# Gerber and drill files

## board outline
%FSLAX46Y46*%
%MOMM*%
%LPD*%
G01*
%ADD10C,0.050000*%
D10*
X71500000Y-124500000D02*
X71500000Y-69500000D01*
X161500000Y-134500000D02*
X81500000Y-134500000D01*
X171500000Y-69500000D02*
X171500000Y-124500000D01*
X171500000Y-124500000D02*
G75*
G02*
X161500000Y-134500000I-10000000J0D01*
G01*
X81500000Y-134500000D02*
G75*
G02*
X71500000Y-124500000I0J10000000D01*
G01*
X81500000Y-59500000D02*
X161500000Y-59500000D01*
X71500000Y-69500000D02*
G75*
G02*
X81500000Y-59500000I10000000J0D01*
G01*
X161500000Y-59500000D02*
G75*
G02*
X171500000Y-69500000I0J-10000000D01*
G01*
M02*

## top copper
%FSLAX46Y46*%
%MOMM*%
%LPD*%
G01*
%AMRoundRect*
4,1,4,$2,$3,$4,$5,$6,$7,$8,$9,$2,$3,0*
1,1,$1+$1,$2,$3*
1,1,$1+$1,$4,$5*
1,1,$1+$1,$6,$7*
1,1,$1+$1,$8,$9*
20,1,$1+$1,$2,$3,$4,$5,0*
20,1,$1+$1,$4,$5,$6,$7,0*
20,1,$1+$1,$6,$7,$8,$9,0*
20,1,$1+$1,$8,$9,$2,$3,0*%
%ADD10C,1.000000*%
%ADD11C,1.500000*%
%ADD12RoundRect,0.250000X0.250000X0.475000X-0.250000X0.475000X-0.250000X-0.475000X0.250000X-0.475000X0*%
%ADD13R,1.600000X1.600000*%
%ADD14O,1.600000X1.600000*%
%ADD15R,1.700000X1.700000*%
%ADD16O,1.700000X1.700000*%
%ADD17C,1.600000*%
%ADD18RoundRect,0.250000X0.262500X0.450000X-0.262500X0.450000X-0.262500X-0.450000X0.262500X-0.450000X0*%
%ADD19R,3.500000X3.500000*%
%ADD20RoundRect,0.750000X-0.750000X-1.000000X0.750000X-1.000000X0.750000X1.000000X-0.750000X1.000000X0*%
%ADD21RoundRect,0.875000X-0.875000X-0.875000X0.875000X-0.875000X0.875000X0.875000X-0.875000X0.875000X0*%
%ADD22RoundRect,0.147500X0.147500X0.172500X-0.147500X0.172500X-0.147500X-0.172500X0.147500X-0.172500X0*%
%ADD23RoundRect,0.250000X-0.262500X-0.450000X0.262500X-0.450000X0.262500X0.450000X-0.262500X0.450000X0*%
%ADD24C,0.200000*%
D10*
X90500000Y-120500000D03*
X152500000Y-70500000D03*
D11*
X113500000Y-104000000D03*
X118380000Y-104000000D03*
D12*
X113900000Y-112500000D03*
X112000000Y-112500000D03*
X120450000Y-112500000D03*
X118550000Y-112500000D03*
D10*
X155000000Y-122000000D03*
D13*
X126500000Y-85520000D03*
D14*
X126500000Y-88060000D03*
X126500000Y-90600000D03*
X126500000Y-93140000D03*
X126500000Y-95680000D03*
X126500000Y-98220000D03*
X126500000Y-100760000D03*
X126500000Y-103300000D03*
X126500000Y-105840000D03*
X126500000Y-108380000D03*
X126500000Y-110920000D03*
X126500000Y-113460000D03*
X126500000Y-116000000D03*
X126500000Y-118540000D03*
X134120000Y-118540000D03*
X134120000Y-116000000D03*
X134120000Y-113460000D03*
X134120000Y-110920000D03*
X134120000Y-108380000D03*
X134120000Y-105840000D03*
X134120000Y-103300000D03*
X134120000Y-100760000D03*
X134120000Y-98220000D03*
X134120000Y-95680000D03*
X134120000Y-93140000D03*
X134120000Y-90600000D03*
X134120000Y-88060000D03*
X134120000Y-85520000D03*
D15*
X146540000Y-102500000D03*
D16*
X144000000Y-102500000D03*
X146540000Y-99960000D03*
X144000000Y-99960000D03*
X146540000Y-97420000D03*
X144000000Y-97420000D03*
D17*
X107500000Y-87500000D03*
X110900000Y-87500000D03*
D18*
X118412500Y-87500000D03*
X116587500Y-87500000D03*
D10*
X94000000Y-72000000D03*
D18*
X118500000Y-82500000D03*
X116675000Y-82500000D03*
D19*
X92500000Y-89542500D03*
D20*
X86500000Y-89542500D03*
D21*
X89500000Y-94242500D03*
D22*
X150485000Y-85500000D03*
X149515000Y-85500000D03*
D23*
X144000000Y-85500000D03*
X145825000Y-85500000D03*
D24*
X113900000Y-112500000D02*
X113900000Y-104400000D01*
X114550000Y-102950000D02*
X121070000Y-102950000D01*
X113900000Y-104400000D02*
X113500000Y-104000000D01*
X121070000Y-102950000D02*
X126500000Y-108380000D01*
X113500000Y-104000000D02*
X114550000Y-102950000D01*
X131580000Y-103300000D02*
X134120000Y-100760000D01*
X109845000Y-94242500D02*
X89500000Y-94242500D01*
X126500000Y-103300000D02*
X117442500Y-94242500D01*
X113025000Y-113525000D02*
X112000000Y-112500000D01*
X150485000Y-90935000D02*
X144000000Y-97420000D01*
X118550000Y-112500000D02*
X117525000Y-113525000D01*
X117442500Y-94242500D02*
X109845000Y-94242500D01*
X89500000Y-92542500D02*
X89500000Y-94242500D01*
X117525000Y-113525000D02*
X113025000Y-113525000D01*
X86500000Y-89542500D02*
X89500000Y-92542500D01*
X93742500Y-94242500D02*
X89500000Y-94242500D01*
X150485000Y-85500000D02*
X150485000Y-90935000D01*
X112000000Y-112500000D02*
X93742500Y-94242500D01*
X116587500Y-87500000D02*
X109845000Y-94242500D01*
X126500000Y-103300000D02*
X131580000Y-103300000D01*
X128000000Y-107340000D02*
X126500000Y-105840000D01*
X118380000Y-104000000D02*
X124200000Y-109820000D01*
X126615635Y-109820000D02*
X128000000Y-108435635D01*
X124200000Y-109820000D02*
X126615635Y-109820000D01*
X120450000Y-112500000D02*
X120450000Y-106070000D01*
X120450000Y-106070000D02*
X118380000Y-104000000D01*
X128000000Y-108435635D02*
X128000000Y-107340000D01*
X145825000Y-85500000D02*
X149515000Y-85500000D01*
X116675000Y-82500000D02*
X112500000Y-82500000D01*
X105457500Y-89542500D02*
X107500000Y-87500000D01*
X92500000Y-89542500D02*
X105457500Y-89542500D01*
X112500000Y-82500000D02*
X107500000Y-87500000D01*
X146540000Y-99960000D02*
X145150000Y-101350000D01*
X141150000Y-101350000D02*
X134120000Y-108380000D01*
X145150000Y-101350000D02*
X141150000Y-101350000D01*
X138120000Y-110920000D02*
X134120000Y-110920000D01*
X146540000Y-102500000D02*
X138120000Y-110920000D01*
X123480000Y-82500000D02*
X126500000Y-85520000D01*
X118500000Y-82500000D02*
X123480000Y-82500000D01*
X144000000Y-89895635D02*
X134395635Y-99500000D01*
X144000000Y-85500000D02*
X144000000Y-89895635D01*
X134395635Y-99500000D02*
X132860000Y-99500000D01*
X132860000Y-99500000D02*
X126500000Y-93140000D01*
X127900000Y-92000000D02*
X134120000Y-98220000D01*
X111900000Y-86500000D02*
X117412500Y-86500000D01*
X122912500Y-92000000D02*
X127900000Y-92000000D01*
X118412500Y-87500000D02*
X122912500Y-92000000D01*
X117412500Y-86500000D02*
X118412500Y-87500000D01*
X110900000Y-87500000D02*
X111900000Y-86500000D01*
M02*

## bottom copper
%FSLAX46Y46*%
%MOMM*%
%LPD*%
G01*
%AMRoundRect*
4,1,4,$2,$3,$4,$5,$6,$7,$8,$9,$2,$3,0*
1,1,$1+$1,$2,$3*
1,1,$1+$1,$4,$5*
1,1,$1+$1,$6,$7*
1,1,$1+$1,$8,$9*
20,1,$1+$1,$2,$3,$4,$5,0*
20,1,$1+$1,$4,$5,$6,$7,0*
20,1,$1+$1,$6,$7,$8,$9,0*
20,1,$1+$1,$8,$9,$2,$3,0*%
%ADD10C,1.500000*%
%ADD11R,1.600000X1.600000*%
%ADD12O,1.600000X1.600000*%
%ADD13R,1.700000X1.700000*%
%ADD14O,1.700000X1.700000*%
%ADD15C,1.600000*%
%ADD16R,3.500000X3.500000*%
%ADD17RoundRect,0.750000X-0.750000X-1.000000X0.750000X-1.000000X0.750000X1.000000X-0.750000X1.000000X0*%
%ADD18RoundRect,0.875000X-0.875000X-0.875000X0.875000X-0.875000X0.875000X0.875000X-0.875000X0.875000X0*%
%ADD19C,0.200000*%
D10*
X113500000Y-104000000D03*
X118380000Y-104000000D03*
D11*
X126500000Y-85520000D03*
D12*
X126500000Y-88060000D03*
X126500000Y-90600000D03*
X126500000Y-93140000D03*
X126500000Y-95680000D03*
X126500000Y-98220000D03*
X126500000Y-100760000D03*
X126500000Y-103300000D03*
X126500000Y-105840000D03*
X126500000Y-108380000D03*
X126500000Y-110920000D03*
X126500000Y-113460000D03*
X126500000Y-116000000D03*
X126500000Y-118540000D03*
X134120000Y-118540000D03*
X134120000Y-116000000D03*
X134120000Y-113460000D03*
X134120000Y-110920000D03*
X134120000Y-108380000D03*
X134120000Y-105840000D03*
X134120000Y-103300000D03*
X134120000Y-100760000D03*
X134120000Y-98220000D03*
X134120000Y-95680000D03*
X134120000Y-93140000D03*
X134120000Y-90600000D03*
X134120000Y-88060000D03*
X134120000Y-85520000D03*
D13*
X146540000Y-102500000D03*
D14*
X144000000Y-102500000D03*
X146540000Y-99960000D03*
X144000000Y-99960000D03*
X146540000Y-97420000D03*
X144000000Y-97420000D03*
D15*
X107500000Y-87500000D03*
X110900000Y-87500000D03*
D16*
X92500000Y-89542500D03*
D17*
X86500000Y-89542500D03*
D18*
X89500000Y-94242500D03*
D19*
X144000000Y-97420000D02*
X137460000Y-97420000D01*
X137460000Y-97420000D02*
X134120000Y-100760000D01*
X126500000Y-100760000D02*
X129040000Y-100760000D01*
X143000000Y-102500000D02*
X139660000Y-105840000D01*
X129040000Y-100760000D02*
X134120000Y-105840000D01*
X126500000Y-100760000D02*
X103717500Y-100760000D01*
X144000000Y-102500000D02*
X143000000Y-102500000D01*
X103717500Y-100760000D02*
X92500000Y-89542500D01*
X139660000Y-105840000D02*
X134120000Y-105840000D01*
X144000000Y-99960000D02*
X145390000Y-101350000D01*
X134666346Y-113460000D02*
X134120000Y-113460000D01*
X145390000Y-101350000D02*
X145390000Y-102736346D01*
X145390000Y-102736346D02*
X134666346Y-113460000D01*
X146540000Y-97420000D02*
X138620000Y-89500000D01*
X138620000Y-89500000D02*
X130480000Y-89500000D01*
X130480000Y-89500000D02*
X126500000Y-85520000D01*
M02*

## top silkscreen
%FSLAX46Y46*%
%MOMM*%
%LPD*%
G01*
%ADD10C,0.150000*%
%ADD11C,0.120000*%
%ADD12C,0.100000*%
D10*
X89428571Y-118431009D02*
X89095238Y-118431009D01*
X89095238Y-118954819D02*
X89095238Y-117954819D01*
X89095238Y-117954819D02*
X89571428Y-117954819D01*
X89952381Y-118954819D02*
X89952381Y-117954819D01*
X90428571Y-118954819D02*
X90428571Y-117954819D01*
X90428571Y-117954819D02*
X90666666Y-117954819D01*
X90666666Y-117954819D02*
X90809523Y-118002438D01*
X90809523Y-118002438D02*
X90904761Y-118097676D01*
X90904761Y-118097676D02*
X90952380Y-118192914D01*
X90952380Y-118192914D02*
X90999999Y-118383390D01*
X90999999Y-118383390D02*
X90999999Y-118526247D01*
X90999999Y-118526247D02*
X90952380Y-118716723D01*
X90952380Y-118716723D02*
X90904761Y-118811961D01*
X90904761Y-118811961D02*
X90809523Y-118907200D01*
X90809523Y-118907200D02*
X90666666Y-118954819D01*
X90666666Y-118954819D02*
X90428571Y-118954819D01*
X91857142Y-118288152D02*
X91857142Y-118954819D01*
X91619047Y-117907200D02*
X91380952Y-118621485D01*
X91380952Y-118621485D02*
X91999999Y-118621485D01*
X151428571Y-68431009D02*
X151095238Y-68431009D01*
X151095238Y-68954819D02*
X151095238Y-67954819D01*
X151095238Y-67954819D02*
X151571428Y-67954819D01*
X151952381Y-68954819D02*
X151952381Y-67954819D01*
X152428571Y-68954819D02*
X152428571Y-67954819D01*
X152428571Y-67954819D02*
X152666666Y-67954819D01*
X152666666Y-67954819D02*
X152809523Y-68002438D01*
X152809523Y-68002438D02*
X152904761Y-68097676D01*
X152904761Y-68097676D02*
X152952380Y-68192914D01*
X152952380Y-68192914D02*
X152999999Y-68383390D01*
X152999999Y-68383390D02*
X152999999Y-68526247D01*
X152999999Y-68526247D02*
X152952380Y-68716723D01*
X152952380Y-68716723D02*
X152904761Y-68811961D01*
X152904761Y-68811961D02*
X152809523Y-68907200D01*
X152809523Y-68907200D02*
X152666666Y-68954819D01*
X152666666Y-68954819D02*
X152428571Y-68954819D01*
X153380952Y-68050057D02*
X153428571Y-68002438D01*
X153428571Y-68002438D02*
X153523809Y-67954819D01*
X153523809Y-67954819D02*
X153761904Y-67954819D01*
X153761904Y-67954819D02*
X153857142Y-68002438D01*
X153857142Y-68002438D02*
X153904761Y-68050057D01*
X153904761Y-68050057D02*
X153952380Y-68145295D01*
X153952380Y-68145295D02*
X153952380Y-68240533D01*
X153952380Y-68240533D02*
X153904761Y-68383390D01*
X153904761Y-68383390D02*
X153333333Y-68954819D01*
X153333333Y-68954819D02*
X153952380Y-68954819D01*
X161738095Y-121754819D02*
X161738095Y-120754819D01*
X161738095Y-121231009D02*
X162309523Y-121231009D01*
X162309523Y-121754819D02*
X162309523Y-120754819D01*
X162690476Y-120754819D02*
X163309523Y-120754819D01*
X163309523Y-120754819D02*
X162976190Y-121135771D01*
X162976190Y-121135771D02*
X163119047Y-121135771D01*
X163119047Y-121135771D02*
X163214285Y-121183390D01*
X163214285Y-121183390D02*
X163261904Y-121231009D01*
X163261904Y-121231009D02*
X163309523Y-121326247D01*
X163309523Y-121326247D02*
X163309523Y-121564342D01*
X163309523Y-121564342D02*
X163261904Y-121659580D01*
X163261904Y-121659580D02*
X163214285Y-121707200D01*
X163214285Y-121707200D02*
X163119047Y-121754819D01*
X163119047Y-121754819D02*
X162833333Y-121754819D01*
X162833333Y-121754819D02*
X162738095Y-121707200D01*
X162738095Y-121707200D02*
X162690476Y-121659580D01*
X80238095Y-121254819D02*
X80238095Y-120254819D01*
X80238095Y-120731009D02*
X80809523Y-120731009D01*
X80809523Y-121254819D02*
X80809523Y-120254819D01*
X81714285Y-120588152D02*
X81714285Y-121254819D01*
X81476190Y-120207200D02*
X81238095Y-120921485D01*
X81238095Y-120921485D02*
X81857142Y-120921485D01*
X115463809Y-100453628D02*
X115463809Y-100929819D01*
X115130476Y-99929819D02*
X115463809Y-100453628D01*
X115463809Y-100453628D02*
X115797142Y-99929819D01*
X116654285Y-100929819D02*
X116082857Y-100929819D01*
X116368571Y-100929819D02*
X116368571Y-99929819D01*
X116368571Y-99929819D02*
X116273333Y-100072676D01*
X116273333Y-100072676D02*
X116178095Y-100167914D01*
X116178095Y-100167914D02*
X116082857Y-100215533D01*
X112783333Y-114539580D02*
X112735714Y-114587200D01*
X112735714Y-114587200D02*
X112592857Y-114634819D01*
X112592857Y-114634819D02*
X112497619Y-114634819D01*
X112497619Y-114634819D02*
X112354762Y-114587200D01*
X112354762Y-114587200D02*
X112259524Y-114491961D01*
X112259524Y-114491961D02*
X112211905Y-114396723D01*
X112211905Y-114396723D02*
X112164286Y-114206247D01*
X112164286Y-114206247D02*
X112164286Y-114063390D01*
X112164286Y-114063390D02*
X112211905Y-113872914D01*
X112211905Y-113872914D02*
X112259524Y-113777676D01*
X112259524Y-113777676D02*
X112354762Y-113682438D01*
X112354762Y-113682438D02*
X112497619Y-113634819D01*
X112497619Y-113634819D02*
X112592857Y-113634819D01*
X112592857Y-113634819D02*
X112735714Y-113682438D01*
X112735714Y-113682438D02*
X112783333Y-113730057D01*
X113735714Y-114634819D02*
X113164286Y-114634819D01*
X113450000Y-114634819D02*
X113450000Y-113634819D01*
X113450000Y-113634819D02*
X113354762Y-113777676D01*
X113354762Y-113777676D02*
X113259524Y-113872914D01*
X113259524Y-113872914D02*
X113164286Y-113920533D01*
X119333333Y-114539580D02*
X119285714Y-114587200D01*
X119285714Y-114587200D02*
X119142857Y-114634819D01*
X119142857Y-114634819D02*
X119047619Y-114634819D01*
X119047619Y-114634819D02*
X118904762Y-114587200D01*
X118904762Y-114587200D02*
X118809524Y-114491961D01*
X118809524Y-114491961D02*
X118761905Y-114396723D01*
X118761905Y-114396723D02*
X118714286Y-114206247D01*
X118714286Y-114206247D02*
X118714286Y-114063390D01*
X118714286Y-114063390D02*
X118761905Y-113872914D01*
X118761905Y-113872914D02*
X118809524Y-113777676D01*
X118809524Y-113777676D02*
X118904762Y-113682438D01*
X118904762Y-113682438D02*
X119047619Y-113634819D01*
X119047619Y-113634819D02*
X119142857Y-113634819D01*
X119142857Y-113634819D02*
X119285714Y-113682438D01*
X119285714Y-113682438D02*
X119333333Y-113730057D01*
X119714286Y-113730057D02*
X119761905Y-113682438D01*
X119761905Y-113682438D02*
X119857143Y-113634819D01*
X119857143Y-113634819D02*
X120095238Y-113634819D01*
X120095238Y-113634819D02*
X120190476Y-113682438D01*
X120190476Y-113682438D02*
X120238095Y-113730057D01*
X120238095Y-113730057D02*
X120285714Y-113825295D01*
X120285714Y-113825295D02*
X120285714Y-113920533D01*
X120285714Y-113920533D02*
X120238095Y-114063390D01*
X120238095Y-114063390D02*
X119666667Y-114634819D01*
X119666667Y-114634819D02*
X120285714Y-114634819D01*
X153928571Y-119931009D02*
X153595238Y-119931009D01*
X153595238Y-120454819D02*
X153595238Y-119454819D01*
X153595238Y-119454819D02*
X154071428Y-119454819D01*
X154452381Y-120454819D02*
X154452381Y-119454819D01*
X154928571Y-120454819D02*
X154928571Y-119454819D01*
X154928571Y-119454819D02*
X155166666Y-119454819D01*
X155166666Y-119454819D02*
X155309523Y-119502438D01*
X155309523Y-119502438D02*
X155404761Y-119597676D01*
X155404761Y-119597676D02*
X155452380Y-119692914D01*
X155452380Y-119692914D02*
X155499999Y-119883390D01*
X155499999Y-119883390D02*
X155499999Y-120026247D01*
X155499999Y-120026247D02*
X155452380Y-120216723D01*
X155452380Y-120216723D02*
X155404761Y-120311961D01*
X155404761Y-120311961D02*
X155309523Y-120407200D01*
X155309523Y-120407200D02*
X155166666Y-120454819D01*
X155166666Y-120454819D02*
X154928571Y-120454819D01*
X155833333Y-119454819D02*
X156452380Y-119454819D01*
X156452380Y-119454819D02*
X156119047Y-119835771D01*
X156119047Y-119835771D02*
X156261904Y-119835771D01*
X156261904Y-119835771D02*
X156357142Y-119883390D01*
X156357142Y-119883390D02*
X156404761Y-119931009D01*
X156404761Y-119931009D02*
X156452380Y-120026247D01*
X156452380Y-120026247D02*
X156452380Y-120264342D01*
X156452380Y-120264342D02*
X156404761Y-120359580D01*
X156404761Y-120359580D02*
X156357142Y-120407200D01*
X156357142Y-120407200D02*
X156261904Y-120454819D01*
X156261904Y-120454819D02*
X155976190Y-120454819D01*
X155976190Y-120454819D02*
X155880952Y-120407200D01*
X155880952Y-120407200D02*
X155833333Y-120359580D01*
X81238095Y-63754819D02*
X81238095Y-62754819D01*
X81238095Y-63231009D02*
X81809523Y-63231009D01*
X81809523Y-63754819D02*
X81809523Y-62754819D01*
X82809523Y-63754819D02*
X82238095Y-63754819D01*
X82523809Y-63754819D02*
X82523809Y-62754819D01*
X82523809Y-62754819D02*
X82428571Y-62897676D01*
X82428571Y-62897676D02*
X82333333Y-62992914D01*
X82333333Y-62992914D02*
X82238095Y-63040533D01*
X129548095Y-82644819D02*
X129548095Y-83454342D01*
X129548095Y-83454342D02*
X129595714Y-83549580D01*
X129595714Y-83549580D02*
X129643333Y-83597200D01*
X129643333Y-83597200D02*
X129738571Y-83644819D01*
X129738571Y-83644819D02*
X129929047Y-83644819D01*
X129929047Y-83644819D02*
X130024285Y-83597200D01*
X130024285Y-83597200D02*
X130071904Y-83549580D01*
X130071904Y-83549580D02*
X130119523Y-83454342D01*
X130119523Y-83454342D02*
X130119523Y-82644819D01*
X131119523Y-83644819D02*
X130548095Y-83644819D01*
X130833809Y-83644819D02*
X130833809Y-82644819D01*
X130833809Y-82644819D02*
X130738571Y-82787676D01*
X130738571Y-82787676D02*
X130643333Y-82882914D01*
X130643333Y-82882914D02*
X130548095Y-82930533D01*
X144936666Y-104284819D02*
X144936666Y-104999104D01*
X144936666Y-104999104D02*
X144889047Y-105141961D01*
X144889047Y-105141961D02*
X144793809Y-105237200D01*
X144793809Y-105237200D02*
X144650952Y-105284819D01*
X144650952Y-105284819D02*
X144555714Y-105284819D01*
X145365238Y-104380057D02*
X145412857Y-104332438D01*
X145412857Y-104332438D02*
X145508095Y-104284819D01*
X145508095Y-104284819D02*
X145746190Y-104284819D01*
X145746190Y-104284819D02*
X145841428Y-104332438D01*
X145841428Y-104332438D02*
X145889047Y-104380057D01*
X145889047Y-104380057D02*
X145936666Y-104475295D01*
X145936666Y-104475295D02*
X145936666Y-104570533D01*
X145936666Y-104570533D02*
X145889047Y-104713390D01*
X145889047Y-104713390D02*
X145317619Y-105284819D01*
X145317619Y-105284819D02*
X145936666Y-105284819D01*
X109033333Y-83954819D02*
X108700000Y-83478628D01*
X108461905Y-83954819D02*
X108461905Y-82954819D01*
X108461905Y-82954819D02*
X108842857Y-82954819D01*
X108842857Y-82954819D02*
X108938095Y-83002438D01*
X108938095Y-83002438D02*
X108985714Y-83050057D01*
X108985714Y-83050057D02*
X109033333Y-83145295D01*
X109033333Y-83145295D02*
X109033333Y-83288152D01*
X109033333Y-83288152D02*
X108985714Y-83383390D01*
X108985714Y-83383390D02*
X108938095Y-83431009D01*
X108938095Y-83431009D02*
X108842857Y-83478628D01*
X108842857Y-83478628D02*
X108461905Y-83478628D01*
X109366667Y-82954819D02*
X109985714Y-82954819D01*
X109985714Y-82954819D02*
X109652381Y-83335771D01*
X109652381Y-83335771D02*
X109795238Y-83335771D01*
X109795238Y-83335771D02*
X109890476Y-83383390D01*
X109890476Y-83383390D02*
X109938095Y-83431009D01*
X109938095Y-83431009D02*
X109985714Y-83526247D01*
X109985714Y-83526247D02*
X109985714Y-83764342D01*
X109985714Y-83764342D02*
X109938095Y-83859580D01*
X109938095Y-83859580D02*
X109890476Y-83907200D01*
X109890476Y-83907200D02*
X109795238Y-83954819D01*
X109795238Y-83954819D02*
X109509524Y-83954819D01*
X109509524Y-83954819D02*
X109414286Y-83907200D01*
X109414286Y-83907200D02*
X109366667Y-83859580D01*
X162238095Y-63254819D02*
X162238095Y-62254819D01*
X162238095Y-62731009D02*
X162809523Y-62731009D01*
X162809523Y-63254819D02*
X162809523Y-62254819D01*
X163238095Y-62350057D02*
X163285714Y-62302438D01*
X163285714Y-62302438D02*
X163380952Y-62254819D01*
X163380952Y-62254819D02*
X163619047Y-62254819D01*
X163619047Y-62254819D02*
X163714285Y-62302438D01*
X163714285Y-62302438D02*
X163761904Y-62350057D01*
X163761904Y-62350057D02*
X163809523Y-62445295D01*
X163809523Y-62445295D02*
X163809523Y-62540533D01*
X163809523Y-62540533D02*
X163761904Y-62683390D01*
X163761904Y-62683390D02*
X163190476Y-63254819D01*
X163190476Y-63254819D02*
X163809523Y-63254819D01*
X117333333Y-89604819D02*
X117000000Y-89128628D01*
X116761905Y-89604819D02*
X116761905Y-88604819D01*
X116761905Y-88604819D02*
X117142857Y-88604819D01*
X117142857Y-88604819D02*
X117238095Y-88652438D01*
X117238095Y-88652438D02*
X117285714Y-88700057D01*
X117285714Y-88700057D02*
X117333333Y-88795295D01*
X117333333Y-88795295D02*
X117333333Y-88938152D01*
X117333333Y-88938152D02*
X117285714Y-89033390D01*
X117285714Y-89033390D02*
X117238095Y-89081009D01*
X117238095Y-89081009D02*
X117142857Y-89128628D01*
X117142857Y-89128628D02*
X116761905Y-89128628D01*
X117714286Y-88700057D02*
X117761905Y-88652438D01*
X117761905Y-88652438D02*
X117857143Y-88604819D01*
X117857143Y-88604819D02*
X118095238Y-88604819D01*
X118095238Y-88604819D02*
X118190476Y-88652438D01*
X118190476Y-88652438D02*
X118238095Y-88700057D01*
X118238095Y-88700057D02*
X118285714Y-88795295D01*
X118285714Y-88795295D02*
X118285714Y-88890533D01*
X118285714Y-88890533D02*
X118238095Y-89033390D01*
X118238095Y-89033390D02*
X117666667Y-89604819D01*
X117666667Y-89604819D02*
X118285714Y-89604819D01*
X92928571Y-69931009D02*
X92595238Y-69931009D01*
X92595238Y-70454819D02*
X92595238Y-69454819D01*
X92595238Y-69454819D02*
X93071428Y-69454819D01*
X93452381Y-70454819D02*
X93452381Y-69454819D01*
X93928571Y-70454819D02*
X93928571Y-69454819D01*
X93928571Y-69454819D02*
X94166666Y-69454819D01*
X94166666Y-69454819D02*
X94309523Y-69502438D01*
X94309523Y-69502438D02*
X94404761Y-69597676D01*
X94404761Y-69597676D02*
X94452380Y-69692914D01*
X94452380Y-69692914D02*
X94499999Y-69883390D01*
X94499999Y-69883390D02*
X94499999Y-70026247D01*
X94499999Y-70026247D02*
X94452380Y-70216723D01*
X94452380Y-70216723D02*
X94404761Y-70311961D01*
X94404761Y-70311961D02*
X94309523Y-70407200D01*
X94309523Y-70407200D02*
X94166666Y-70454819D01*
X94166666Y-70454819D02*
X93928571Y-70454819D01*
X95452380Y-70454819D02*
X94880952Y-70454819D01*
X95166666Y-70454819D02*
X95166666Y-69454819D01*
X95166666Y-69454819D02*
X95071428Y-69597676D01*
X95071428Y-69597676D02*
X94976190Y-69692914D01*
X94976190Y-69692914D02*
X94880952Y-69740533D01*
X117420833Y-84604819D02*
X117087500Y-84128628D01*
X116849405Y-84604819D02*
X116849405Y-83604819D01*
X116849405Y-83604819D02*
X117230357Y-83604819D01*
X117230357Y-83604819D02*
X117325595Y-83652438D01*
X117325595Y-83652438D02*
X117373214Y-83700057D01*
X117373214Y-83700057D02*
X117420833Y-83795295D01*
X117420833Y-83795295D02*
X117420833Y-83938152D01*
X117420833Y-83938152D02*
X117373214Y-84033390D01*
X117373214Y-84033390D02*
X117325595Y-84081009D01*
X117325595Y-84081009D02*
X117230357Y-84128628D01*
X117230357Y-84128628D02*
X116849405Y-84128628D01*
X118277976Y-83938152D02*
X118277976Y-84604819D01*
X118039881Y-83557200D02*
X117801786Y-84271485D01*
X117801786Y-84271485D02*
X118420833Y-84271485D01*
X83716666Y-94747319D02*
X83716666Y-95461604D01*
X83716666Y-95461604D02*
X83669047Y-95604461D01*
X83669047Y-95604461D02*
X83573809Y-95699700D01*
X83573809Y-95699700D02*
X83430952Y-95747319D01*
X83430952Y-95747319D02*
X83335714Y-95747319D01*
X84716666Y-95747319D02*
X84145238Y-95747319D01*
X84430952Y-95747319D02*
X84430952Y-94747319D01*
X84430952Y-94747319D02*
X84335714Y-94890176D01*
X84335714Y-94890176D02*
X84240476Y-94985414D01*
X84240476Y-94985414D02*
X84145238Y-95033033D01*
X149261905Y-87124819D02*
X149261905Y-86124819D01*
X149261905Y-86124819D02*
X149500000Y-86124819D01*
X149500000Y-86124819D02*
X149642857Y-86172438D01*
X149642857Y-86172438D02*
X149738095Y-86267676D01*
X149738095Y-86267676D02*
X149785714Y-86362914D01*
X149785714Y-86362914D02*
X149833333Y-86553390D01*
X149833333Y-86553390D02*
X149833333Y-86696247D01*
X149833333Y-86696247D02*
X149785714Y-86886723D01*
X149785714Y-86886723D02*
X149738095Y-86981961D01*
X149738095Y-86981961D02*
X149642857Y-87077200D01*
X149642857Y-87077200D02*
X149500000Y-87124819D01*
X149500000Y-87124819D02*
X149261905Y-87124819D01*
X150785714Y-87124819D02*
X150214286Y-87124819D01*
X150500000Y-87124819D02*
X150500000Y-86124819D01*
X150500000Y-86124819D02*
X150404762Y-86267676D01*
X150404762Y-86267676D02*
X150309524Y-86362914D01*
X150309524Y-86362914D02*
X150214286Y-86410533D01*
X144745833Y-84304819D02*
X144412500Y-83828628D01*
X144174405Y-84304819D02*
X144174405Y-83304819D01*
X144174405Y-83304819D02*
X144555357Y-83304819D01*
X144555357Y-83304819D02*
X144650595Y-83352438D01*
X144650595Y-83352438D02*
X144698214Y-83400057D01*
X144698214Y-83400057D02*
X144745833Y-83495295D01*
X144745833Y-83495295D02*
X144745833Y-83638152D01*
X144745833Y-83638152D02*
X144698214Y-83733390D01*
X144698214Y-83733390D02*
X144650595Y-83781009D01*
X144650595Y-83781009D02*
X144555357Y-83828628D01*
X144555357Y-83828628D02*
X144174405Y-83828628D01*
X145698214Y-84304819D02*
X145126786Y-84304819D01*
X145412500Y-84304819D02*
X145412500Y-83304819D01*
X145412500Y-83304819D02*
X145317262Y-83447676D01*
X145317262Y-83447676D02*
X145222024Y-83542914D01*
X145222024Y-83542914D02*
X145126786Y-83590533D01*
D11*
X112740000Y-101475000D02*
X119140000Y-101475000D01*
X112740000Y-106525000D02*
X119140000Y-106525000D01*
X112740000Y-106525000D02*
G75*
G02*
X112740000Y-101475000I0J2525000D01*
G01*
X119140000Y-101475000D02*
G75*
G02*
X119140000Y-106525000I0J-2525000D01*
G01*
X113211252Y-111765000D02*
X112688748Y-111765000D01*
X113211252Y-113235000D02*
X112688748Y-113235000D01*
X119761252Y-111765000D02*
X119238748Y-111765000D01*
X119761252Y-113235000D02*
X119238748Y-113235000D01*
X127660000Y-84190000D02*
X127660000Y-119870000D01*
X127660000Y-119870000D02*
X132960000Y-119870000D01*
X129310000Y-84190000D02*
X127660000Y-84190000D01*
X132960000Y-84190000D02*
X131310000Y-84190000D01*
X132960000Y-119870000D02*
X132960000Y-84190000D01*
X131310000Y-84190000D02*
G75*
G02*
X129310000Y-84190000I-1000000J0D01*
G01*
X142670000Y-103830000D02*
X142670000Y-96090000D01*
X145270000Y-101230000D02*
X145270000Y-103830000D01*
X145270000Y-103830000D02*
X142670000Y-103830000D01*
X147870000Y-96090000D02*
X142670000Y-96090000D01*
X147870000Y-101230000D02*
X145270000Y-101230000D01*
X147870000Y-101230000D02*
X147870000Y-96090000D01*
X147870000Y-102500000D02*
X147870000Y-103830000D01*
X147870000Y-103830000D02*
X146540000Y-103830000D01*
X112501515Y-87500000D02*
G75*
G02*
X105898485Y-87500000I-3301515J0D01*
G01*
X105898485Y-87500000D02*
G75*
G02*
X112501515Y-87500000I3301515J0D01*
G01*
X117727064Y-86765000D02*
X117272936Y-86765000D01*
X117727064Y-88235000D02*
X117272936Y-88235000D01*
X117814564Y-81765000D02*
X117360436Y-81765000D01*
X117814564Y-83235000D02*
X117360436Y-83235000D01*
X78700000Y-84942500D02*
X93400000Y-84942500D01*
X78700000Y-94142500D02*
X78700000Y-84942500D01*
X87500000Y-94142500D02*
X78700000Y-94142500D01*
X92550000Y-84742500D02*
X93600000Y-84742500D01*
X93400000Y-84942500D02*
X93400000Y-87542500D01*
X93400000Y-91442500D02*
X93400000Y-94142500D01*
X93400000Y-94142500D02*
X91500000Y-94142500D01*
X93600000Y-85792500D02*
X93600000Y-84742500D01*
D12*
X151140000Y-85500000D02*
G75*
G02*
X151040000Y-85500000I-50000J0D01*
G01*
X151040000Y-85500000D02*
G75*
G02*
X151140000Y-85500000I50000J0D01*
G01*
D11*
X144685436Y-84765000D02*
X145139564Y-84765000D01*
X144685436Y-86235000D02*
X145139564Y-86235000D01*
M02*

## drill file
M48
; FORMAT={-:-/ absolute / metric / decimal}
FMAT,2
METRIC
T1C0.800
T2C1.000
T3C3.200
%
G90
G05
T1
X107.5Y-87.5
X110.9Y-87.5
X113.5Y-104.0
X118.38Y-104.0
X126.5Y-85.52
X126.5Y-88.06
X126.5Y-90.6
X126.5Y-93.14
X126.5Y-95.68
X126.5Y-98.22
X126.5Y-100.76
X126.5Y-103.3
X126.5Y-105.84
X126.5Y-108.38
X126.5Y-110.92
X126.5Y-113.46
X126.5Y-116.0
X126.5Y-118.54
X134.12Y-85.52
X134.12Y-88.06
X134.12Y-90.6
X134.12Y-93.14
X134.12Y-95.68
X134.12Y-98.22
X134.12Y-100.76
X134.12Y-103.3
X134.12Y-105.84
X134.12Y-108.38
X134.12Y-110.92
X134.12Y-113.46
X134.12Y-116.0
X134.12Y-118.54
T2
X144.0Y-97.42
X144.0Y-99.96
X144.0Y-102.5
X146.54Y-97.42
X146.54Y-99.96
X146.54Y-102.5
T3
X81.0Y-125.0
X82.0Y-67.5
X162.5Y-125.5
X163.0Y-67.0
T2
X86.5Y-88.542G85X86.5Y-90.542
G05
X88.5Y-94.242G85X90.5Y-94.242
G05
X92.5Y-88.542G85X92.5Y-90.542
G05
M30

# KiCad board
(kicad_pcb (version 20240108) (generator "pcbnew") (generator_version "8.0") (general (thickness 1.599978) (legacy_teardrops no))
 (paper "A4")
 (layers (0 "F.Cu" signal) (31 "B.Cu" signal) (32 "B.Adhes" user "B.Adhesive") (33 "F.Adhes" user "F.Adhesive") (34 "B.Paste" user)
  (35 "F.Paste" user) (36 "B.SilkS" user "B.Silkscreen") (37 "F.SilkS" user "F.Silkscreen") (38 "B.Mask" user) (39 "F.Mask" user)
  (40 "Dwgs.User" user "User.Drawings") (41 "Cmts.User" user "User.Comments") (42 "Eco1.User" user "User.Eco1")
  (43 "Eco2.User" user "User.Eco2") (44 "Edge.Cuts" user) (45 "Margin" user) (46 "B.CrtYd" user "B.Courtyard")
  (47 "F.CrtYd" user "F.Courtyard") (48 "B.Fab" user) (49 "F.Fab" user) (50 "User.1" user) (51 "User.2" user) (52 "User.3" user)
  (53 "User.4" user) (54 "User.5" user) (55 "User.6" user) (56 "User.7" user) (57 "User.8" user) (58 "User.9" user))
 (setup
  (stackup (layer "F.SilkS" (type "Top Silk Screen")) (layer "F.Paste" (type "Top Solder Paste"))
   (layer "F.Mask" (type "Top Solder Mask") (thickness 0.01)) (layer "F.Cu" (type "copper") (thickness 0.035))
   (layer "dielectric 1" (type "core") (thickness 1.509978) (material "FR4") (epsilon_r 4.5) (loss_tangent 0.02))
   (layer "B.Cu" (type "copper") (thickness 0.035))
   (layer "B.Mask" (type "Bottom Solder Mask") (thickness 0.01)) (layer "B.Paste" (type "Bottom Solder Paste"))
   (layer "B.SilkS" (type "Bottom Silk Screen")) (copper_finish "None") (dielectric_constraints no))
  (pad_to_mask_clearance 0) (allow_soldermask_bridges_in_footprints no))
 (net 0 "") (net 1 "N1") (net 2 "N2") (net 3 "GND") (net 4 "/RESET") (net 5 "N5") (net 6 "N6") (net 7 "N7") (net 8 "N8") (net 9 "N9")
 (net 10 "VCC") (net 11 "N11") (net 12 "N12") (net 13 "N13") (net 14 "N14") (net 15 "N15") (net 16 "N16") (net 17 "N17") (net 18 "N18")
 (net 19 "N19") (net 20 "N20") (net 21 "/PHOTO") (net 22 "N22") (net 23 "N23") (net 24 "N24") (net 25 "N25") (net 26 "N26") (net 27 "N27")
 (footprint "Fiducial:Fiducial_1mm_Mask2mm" (layer "F.Cu") (at 90.5 120.5)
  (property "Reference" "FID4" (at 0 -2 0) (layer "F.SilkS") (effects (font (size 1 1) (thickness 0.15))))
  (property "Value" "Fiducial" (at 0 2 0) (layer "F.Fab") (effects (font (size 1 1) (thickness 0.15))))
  (pad "" smd circle (at 0 0) (size 1 1) (layers "F.Cu" "F.Mask") (solder_mask_margin 0.5) (clearance 0.5)))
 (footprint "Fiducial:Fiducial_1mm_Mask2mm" (layer "F.Cu") (at 152.5 70.5)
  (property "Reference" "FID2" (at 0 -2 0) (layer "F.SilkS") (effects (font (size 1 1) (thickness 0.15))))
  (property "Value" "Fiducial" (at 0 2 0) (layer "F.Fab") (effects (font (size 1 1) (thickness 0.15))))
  (pad "" smd circle (at 0 0) (size 1 1) (layers "F.Cu" "F.Mask") (solder_mask_margin 0.5) (clearance 0.5)))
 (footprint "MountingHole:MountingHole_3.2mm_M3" (layer "F.Cu") (at 162.5 125.5)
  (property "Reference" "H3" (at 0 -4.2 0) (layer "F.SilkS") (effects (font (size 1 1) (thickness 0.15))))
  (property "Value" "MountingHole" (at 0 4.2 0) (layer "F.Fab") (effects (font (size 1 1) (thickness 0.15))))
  (pad "" np_thru_hole circle (at 0 0) (size 3.2 3.2) (drill 3.2) (layers "*.Cu" "*.Mask")))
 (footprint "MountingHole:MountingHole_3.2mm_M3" (layer "F.Cu") (at 81 125)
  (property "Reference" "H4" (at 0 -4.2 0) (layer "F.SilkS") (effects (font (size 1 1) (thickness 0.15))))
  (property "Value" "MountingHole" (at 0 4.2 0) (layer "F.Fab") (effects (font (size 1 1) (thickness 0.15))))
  (pad "" np_thru_hole circle (at 0 0) (size 3.2 3.2) (drill 3.2) (layers "*.Cu" "*.Mask")))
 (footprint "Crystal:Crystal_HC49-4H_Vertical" (layer "F.Cu") (at 113.5 104)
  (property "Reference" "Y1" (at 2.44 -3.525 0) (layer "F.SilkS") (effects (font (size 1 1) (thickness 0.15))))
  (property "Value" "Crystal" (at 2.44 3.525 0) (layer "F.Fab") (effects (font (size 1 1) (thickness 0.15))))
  (fp_line (start -0.76 -2.525) (end 5.64 -2.525) (stroke (width 0.12) (type solid)) (layer "F.SilkS"))
  (fp_line (start -0.76 2.525) (end 5.64 2.525) (stroke (width 0.12) (type solid)) (layer "F.SilkS"))
  (fp_arc (start -0.76 2.525) (mid -3.285 0) (end -0.76 -2.525) (stroke (width 0.12) (type solid)) (layer "F.SilkS"))
  (fp_arc (start 5.64 -2.525) (mid 8.165 0) (end 5.64 2.525) (stroke (width 0.12) (type solid)) (layer "F.SilkS"))
  (pad "1" thru_hole circle (at 0 0) (size 1.5 1.5) (drill 0.8) (layers "*.Cu" "*.Mask") (remove_unused_layers no) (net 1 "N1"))
  (pad "2" thru_hole circle (at 4.88 0) (size 1.5 1.5) (drill 0.8) (layers "*.Cu" "*.Mask") (remove_unused_layers no) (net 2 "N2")))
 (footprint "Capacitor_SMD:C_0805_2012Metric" (layer "F.Cu") (at 112.95 112.5 180)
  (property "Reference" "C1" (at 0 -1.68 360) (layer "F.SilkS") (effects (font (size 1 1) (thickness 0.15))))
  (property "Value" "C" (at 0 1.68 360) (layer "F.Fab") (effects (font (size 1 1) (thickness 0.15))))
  (fp_line (start -0.261252 0.735) (end 0.261252 0.735) (stroke (width 0.12) (type solid)) (layer "F.SilkS"))
  (fp_line (start -0.261252 -0.735) (end 0.261252 -0.735) (stroke (width 0.12) (type solid)) (layer "F.SilkS"))
  (pad "1" smd roundrect (at -0.95 0 180) (size 1 1.45) (layers "F.Cu" "F.Paste" "F.Mask") (roundrect_rratio 0.25) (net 1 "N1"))
  (pad "2" smd roundrect (at 0.95 0 180) (size 1 1.45) (layers "F.Cu" "F.Paste" "F.Mask") (roundrect_rratio 0.25) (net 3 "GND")))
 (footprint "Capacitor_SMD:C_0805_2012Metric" (layer "F.Cu") (at 119.5 112.5 180)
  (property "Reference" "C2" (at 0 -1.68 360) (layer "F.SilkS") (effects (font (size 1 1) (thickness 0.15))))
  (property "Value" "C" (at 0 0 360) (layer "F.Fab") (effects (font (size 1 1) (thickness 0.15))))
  (fp_line (start -0.261252 0.735) (end 0.261252 0.735) (stroke (width 0.12) (type solid)) (layer "F.SilkS"))
  (fp_line (start -0.261252 -0.735) (end 0.261252 -0.735) (stroke (width 0.12) (type solid)) (layer "F.SilkS"))
  (pad "1" smd roundrect (at -0.95 0 180) (size 1 1.45) (layers "F.Cu" "F.Paste" "F.Mask") (roundrect_rratio 0.25) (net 2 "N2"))
  (pad "2" smd roundrect (at 0.95 0 180) (size 1 1.45) (layers "F.Cu" "F.Paste" "F.Mask") (roundrect_rratio 0.25) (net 3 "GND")))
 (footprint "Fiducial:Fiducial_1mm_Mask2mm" (layer "F.Cu") (at 155 122)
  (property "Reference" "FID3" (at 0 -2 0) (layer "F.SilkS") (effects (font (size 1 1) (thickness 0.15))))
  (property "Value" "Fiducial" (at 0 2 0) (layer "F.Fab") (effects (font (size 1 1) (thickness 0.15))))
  (pad "" smd circle (at 0 0) (size 1 1) (layers "F.Cu" "F.Mask") (solder_mask_margin 0.5) (clearance 0.5)))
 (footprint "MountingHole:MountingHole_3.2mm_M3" (layer "F.Cu") (at 82 67.5)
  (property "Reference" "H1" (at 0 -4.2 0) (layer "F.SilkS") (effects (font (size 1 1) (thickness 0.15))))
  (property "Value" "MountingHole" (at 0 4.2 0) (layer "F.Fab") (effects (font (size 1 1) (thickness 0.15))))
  (pad "" np_thru_hole circle (at 0 0) (size 3.2 3.2) (drill 3.2) (layers "*.Cu" "*.Mask")))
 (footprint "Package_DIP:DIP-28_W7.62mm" (layer "F.Cu") (at 126.5 85.52)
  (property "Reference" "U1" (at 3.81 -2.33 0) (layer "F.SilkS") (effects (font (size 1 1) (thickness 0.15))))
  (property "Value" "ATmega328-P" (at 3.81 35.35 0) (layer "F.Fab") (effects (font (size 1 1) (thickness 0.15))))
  (fp_line (start 1.16 -1.33) (end 1.16 34.35) (stroke (width 0.12) (type solid)) (layer "F.SilkS"))
  (fp_line (start 1.16 34.35) (end 6.46 34.35) (stroke (width 0.12) (type solid)) (layer "F.SilkS"))
  (fp_line (start 2.81 -1.33) (end 1.16 -1.33) (stroke (width 0.12) (type solid)) (layer "F.SilkS"))
  (fp_line (start 6.46 -1.33) (end 4.81 -1.33) (stroke (width 0.12) (type solid)) (layer "F.SilkS"))
  (fp_line (start 6.46 34.35) (end 6.46 -1.33) (stroke (width 0.12) (type solid)) (layer "F.SilkS"))
  (fp_arc (start 4.81 -1.33) (mid 3.81 -0.33) (end 2.81 -1.33) (stroke (width 0.12) (type solid)) (layer "F.SilkS"))
  (pad "1" thru_hole rect (at 0 0) (size 1.6 1.6) (drill 0.8) (layers "*.Cu" "*.Mask") (remove_unused_layers no) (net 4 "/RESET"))
  (pad "2" thru_hole oval (at 0 2.54) (size 1.6 1.6) (drill 0.8) (layers "*.Cu" "*.Mask") (remove_unused_layers no) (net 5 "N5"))
  (pad "3" thru_hole oval (at 0 5.08) (size 1.6 1.6) (drill 0.8) (layers "*.Cu" "*.Mask") (remove_unused_layers no) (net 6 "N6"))
  (pad "4" thru_hole oval (at 0 7.62) (size 1.6 1.6) (drill 0.8) (layers "*.Cu" "*.Mask") (remove_unused_layers no) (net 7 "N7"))
  (pad "5" thru_hole oval (at 0 10.16) (size 1.6 1.6) (drill 0.8) (layers "*.Cu" "*.Mask") (remove_unused_layers no) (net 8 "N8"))
  (pad "6" thru_hole oval (at 0 12.7) (size 1.6 1.6) (drill 0.8) (layers "*.Cu" "*.Mask") (remove_unused_layers no) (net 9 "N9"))
  (pad "7" thru_hole oval (at 0 15.24) (size 1.6 1.6) (drill 0.8) (layers "*.Cu" "*.Mask") (remove_unused_layers no) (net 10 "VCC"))
  (pad "8" thru_hole oval (at 0 17.78) (size 1.6 1.6) (drill 0.8) (layers "*.Cu" "*.Mask") (remove_unused_layers no) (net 3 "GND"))
  (pad "9" thru_hole oval (at 0 20.32) (size 1.6 1.6) (drill 0.8) (layers "*.Cu" "*.Mask") (remove_unused_layers no) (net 2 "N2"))
  (pad "10" thru_hole oval (at 0 22.86) (size 1.6 1.6) (drill 0.8) (layers "*.Cu" "*.Mask") (remove_unused_layers no) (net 1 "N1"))
  (pad "11" thru_hole oval (at 0 25.4) (size 1.6 1.6) (drill 0.8) (layers "*.Cu" "*.Mask") (remove_unused_layers no) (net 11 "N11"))
  (pad "12" thru_hole oval (at 0 27.94) (size 1.6 1.6) (drill 0.8) (layers "*.Cu" "*.Mask") (remove_unused_layers no) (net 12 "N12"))
  (pad "13" thru_hole oval (at 0 30.48) (size 1.6 1.6) (drill 0.8) (layers "*.Cu" "*.Mask") (remove_unused_layers no) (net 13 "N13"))
  (pad "14" thru_hole oval (at 0 33.02) (size 1.6 1.6) (drill 0.8) (layers "*.Cu" "*.Mask") (remove_unused_layers no) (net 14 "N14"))
  (pad "15" thru_hole oval (at 7.62 33.02) (size 1.6 1.6) (drill 0.8) (layers "*.Cu" "*.Mask") (remove_unused_layers no) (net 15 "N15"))
  (pad "16" thru_hole oval (at 7.62 30.48) (size 1.6 1.6) (drill 0.8) (layers "*.Cu" "*.Mask") (remove_unused_layers no) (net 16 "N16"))
  (pad "17" thru_hole oval (at 7.62 27.94) (size 1.6 1.6) (drill 0.8) (layers "*.Cu" "*.Mask") (remove_unused_layers no) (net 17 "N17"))
  (pad "18" thru_hole oval (at 7.62 25.4) (size 1.6 1.6) (drill 0.8) (layers "*.Cu" "*.Mask") (remove_unused_layers no) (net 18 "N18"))
  (pad "19" thru_hole oval (at 7.62 22.86) (size 1.6 1.6) (drill 0.8) (layers "*.Cu" "*.Mask") (remove_unused_layers no) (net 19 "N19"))
  (pad "20" thru_hole oval (at 7.62 20.32) (size 1.6 1.6) (drill 0.8) (layers "*.Cu" "*.Mask") (remove_unused_layers no) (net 10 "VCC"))
  (pad "21" thru_hole oval (at 7.62 17.78) (size 1.6 1.6) (drill 0.8) (layers "*.Cu" "*.Mask") (remove_unused_layers no) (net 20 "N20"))
  (pad "22" thru_hole oval (at 7.62 15.24) (size 1.6 1.6) (drill 0.8) (layers "*.Cu" "*.Mask") (remove_unused_layers no) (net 3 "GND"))
  (pad "23" thru_hole oval (at 7.62 12.7) (size 1.6 1.6) (drill 0.8) (layers "*.Cu" "*.Mask") (remove_unused_layers no) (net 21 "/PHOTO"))
  (pad "24" thru_hole oval (at 7.62 10.16) (size 1.6 1.6) (drill 0.8) (layers "*.Cu" "*.Mask") (remove_unused_layers no) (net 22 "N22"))
  (pad "25" thru_hole oval (at 7.62 7.62) (size 1.6 1.6) (drill 0.8) (layers "*.Cu" "*.Mask") (remove_unused_layers no) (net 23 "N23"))
  (pad "26" thru_hole oval (at 7.62 5.08) (size 1.6 1.6) (drill 0.8) (layers "*.Cu" "*.Mask") (remove_unused_layers no) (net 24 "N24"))
  (pad "27" thru_hole oval (at 7.62 2.54) (size 1.6 1.6) (drill 0.8) (layers "*.Cu" "*.Mask") (remove_unused_layers no) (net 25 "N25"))
  (pad "28" thru_hole oval (at 7.62 0) (size 1.6 1.6) (drill 0.8) (layers "*.Cu" "*.Mask") (remove_unused_layers no) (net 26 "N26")))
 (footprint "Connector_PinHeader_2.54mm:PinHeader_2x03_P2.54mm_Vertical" (layer "F.Cu") (at 146.54 102.5 180)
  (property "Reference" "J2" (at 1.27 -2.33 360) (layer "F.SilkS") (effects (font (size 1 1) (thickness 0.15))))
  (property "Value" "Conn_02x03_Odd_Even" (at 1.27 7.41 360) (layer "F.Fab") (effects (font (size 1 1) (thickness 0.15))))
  (fp_line (start 3.87 -1.33) (end 3.87 6.41) (stroke (width 0.12) (type solid)) (layer "F.SilkS"))
  (fp_line (start 1.27 1.27) (end 1.27 -1.33) (stroke (width 0.12) (type solid)) (layer "F.SilkS"))
  (fp_line (start 1.27 -1.33) (end 3.87 -1.33) (stroke (width 0.12) (type solid)) (layer "F.SilkS"))
  (fp_line (start -1.33 6.41) (end 3.87 6.41) (stroke (width 0.12) (type solid)) (layer "F.SilkS"))
  (fp_line (start -1.33 1.27) (end 1.27 1.27) (stroke (width 0.12) (type solid)) (layer "F.SilkS"))
  (fp_line (start -1.33 1.27) (end -1.33 6.41) (stroke (width 0.12) (type solid)) (layer "F.SilkS"))
  (fp_line (start -1.33 0) (end -1.33 -1.33) (stroke (width 0.12) (type solid)) (layer "F.SilkS"))
  (fp_line (start -1.33 -1.33) (end 0 -1.33) (stroke (width 0.12) (type solid)) (layer "F.SilkS"))
  (pad "1" thru_hole rect (at 0 0 180) (size 1.7 1.7) (drill 1) (layers "*.Cu" "*.Mask") (remove_unused_layers no) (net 18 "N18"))
  (pad "2" thru_hole oval (at 2.54 0 180) (size 1.7 1.7) (drill 1) (layers "*.Cu" "*.Mask") (remove_unused_layers no) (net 10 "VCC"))
  (pad "3" thru_hole oval (at 0 2.54 180) (size 1.7 1.7) (drill 1) (layers "*.Cu" "*.Mask") (remove_unused_layers no) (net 19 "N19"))
  (pad "4" thru_hole oval (at 2.54 2.54 180) (size 1.7 1.7) (drill 1) (layers "*.Cu" "*.Mask") (remove_unused_layers no) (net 17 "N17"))
  (pad "5" thru_hole oval (at 0 5.08 180) (size 1.7 1.7) (drill 1) (layers "*.Cu" "*.Mask") (remove_unused_layers no) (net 4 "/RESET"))
  (pad "6" thru_hole oval (at 2.54 5.08 180) (size 1.7 1.7) (drill 1) (layers "*.Cu" "*.Mask") (remove_unused_layers no) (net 3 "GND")))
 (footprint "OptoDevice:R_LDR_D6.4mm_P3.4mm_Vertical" (layer "F.Cu") (at 107.5 87.5)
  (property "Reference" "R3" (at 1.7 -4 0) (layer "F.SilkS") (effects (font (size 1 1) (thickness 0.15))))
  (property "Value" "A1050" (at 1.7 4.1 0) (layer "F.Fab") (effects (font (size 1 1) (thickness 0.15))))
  (fp_circle (center 1.7 0) (end 5 -0.1) (stroke (width 0.12) (type solid)) (fill none) (layer "F.SilkS"))
  (pad "1" thru_hole circle (at 0 0) (size 1.6 1.6) (drill 0.8) (layers "*.Cu" "*.Mask") (remove_unused_layers no) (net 10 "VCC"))
  (pad "2" thru_hole circle (at 3.4 0) (size 1.6 1.6) (drill 0.8) (layers "*.Cu" "*.Mask") (remove_unused_layers no) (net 21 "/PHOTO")))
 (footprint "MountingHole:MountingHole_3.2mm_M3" (layer "F.Cu") (at 163 67)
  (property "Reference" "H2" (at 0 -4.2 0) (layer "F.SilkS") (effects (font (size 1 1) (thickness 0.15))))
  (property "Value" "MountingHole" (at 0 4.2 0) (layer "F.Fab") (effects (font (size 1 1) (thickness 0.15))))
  (pad "" np_thru_hole circle (at 0 0) (size 3.2 3.2) (drill 3.2) (layers "*.Cu" "*.Mask")))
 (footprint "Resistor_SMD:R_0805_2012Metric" (layer "F.Cu") (at 117.5 87.5 180)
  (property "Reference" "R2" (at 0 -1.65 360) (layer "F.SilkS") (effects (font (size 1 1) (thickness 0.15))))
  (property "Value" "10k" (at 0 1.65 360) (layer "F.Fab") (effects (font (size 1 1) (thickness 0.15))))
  (fp_line (start -0.227064 0.735) (end 0.227064 0.735) (stroke (width 0.12) (type solid)) (layer "F.SilkS"))
  (fp_line (start -0.227064 -0.735) (end 0.227064 -0.735) (stroke (width 0.12) (type solid)) (layer "F.SilkS"))
  (pad "1" smd roundrect (at -0.9125 0 180) (size 1.025 1.4) (layers "F.Cu" "F.Paste" "F.Mask") (roundrect_rratio 0.243902)
   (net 21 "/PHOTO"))
  (pad "2" smd roundrect (at 0.9125 0 180) (size 1.025 1.4) (layers "F.Cu" "F.Paste" "F.Mask") (roundrect_rratio 0.243902) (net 3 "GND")))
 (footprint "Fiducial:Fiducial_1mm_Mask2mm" (layer "F.Cu") (at 94 72)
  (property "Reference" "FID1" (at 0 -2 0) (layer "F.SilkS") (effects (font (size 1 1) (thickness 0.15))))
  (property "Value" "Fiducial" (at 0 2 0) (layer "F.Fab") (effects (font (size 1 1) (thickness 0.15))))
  (pad "" smd circle (at 0 0) (size 1 1) (layers "F.Cu" "F.Mask") (solder_mask_margin 0.5) (clearance 0.5)))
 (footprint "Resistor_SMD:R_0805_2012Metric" (layer "F.Cu") (at 117.5875 82.5 180)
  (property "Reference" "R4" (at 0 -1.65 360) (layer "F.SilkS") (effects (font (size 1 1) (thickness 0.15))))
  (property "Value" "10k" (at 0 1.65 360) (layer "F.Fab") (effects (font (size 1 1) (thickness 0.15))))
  (fp_line (start -0.227064 0.735) (end 0.227064 0.735) (stroke (width 0.12) (type solid)) (layer "F.SilkS"))
  (fp_line (start -0.227064 -0.735) (end 0.227064 -0.735) (stroke (width 0.12) (type solid)) (layer "F.SilkS"))
  (pad "1" smd roundrect (at -0.9125 0 180) (size 1.025 1.4) (layers "F.Cu" "F.Paste" "F.Mask") (roundrect_rratio 0.243902) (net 4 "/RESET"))
  (pad "2" smd roundrect (at 0.9125 0 180) (size 1.025 1.4) (layers "F.Cu" "F.Paste" "F.Mask") (roundrect_rratio 0.243902) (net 10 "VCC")))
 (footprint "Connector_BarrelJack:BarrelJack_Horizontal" (layer "F.Cu") (at 92.5 89.5425)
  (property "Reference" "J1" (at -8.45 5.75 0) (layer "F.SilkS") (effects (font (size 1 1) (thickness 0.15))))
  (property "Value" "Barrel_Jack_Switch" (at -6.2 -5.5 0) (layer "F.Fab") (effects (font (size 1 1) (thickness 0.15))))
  (fp_line (start -13.8 -4.6) (end 0.9 -4.6) (stroke (width 0.12) (type solid)) (layer "F.SilkS"))
  (fp_line (start -13.8 4.6) (end -13.8 -4.6) (stroke (width 0.12) (type solid)) (layer "F.SilkS"))
  (fp_line (start -5 4.6) (end -13.8 4.6) (stroke (width 0.12) (type solid)) (layer "F.SilkS"))
  (fp_line (start 0.05 -4.8) (end 1.1 -4.8) (stroke (width 0.12) (type solid)) (layer "F.SilkS"))
  (fp_line (start 0.9 -4.6) (end 0.9 -2) (stroke (width 0.12) (type solid)) (layer "F.SilkS"))
  (fp_line (start 0.9 1.9) (end 0.9 4.6) (stroke (width 0.12) (type solid)) (layer "F.SilkS"))
  (fp_line (start 0.9 4.6) (end -1 4.6) (stroke (width 0.12) (type solid)) (layer "F.SilkS"))
  (fp_line (start 1.1 -3.75) (end 1.1 -4.8) (stroke (width 0.12) (type solid)) (layer "F.SilkS"))
  (pad "1" thru_hole rect (at 0 0) (size 3.5 3.5) (drill oval 1 3) (layers "*.Cu" "*.Mask") (remove_unused_layers no) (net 10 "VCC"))
  (pad "2" thru_hole roundrect (at -6 0) (size 3 3.5) (drill oval 1 3) (layers "*.Cu" "*.Mask") (remove_unused_layers no)
   (roundrect_rratio 0.25) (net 3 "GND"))
  (pad "3" thru_hole roundrect (at -3 4.7) (size 3.5 3.5) (drill oval 3 1) (layers "*.Cu" "*.Mask") (remove_unused_layers no)
   (roundrect_rratio 0.25) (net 3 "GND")))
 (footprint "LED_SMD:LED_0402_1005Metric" (layer "F.Cu") (at 150 85.5 180)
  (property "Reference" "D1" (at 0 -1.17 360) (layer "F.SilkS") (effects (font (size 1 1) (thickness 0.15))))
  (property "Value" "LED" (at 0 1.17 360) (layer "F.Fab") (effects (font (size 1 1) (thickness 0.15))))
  (fp_circle (center -1.09 0) (end -1.04 0) (stroke (width 0.1) (type solid)) (fill none) (layer "F.SilkS"))
  (pad "1" smd roundrect (at -0.485 0 180) (size 0.59 0.64) (layers "F.Cu" "F.Paste" "F.Mask") (roundrect_rratio 0.25) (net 3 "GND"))
  (pad "2" smd roundrect (at 0.485 0 180) (size 0.59 0.64) (layers "F.Cu" "F.Paste" "F.Mask") (roundrect_rratio 0.25) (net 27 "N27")))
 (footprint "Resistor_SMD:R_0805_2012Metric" (layer "F.Cu") (at 144.9125 85.5)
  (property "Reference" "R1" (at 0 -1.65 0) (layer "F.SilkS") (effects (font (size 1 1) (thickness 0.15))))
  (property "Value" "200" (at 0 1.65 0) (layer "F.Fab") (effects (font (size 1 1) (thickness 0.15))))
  (fp_line (start -0.227064 -0.735) (end 0.227064 -0.735) (stroke (width 0.12) (type solid)) (layer "F.SilkS"))
  (fp_line (start -0.227064 0.735) (end 0.227064 0.735) (stroke (width 0.12) (type solid)) (layer "F.SilkS"))
  (pad "1" smd roundrect (at -0.9125 0) (size 1.025 1.4) (layers "F.Cu" "F.Paste" "F.Mask") (roundrect_rratio 0.243902) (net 7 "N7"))
  (pad "2" smd roundrect (at 0.9125 0) (size 1.025 1.4) (layers "F.Cu" "F.Paste" "F.Mask") (roundrect_rratio 0.243902) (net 27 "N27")))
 (gr_line (start 71.5 124.5) (end 71.5 69.5) (stroke (width 0.05) (type default)) (layer "Edge.Cuts"))
 (gr_line (start 161.5 134.5) (end 81.5 134.5) (stroke (width 0.05) (type default)) (layer "Edge.Cuts"))
 (gr_line (start 171.5 69.5) (end 171.5 124.5) (stroke (width 0.05) (type default)) (layer "Edge.Cuts"))
 (gr_arc (start 171.5 124.5) (mid 168.571068 131.571068) (end 161.5 134.5) (stroke (width 0.05) (type default)) (layer "Edge.Cuts"))
 (gr_arc (start 81.5 134.5) (mid 74.428932 131.571068) (end 71.5 124.5) (stroke (width 0.05) (type default)) (layer "Edge.Cuts"))
 (gr_line (start 81.5 59.5) (end 161.5 59.5) (stroke (width 0.05) (type default)) (layer "Edge.Cuts"))
 (gr_arc (start 71.5 69.5) (mid 74.428932 62.428932) (end 81.5 59.5) (stroke (width 0.05) (type default)) (layer "Edge.Cuts"))
 (gr_arc (start 161.5 59.5) (mid 168.571068 62.428932) (end 171.5 69.5) (stroke (width 0.05) (type default)) (layer "Edge.Cuts"))
 (segment (start 113.9 112.5) (end 113.9 104.4) (width 0.2) (layer "F.Cu") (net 1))
 (segment (start 114.55 102.95) (end 121.07 102.95) (width 0.2) (layer "F.Cu") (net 1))
 (segment (start 113.9 104.4) (end 113.5 104) (width 0.2) (layer "F.Cu") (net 1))
 (segment (start 121.07 102.95) (end 126.5 108.38) (width 0.2) (layer "F.Cu") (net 1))
 (segment (start 113.5 104) (end 114.55 102.95) (width 0.2) (layer "F.Cu") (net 1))
 (segment (start 131.58 103.3) (end 134.12 100.76) (width 0.2) (layer "F.Cu") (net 3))
 (segment (start 109.845 94.2425) (end 89.5 94.2425) (width 0.2) (layer "F.Cu") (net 3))
 (segment (start 126.5 103.3) (end 117.4425 94.2425) (width 0.2) (layer "F.Cu") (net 3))
 (segment (start 113.025 113.525) (end 112 112.5) (width 0.2) (layer "F.Cu") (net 3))
 (segment (start 150.485 90.935) (end 144 97.42) (width 0.2) (layer "F.Cu") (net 3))
 (segment (start 118.55 112.5) (end 117.525 113.525) (width 0.2) (layer "F.Cu") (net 3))
 (segment (start 117.4425 94.2425) (end 109.845 94.2425) (width 0.2) (layer "F.Cu") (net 3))
 (segment (start 89.5 92.5425) (end 89.5 94.2425) (width 0.2) (layer "F.Cu") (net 3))
 (segment (start 117.525 113.525) (end 113.025 113.525) (width 0.2) (layer "F.Cu") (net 3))
 (segment (start 86.5 89.5425) (end 89.5 92.5425) (width 0.2) (layer "F.Cu") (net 3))
 (segment (start 93.7425 94.2425) (end 89.5 94.2425) (width 0.2) (layer "F.Cu") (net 3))
 (segment (start 150.485 85.5) (end 150.485 90.935) (width 0.2) (layer "F.Cu") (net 3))
 (segment (start 112 112.5) (end 93.7425 94.2425) (width 0.2) (layer "F.Cu") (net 3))
 (segment (start 116.5875 87.5) (end 109.845 94.2425) (width 0.2) (layer "F.Cu") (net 3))
 (segment (start 126.5 103.3) (end 131.58 103.3) (width 0.2) (layer "F.Cu") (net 3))
 (segment (start 144 97.42) (end 137.46 97.42) (width 0.2) (layer "B.Cu") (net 3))
 (segment (start 137.46 97.42) (end 134.12 100.76) (width 0.2) (layer "B.Cu") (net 3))
 (segment (start 128 107.34) (end 126.5 105.84) (width 0.2) (layer "F.Cu") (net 2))
 (segment (start 118.38 104) (end 124.2 109.82) (width 0.2) (layer "F.Cu") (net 2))
 (segment (start 126.615635 109.82) (end 128 108.435635) (width 0.2) (layer "F.Cu") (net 2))
 (segment (start 124.2 109.82) (end 126.615635 109.82) (width 0.2) (layer "F.Cu") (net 2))
 (segment (start 120.45 112.5) (end 120.45 106.07) (width 0.2) (layer "F.Cu") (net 2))
 (segment (start 120.45 106.07) (end 118.38 104) (width 0.2) (layer "F.Cu") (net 2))
 (segment (start 128 108.435635) (end 128 107.34) (width 0.2) (layer "F.Cu") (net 2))
 (segment (start 145.825 85.5) (end 149.515 85.5) (width 0.2) (layer "F.Cu") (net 27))
 (segment (start 116.675 82.5) (end 112.5 82.5) (width 0.2) (layer "F.Cu") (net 10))
 (segment (start 105.4575 89.5425) (end 107.5 87.5) (width 0.2) (layer "F.Cu") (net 10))
 (segment (start 92.5 89.5425) (end 105.4575 89.5425) (width 0.2) (layer "F.Cu") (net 10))
 (segment (start 112.5 82.5) (end 107.5 87.5) (width 0.2) (layer "F.Cu") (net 10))
 (segment (start 126.5 100.76) (end 129.04 100.76) (width 0.2) (layer "B.Cu") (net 10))
 (segment (start 143 102.5) (end 139.66 105.84) (width 0.2) (layer "B.Cu") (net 10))
 (segment (start 129.04 100.76) (end 134.12 105.84) (width 0.2) (layer "B.Cu") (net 10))
 (segment (start 126.5 100.76) (end 103.7175 100.76) (width 0.2) (layer "B.Cu") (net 10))
 (segment (start 144 102.5) (end 143 102.5) (width 0.2) (layer "B.Cu") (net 10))
 (segment (start 103.7175 100.76) (end 92.5 89.5425) (width 0.2) (layer "B.Cu") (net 10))
 (segment (start 139.66 105.84) (end 134.12 105.84) (width 0.2) (layer "B.Cu") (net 10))
 (segment (start 144 99.96) (end 145.39 101.35) (width 0.2) (layer "B.Cu") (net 17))
 (segment (start 134.666346 113.46) (end 134.12 113.46) (width 0.2) (layer "B.Cu") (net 17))
 (segment (start 145.39 101.35) (end 145.39 102.736346) (width 0.2) (layer "B.Cu") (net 17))
 (segment (start 145.39 102.736346) (end 134.666346 113.46) (width 0.2) (layer "B.Cu") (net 17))
 (segment (start 146.54 99.96) (end 145.15 101.35) (width 0.2) (layer "F.Cu") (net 19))
 (segment (start 141.15 101.35) (end 134.12 108.38) (width 0.2) (layer "F.Cu") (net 19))
 (segment (start 145.15 101.35) (end 141.15 101.35) (width 0.2) (layer "F.Cu") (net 19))
 (segment (start 138.12 110.92) (end 134.12 110.92) (width 0.2) (layer "F.Cu") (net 18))
 (segment (start 146.54 102.5) (end 138.12 110.92) (width 0.2) (layer "F.Cu") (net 18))
 (segment (start 123.48 82.5) (end 126.5 85.52) (width 0.2) (layer "F.Cu") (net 4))
 (segment (start 118.5 82.5) (end 123.48 82.5) (width 0.2) (layer "F.Cu") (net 4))
 (segment (start 146.54 97.42) (end 138.62 89.5) (width 0.2) (layer "B.Cu") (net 4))
 (segment (start 138.62 89.5) (end 130.48 89.5) (width 0.2) (layer "B.Cu") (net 4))
 (segment (start 130.48 89.5) (end 126.5 85.52) (width 0.2) (layer "B.Cu") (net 4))
 (segment (start 144 89.895635) (end 134.395635 99.5) (width 0.2) (layer "F.Cu") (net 7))
 (segment (start 144 85.5) (end 144 89.895635) (width 0.2) (layer "F.Cu") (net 7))
 (segment (start 134.395635 99.5) (end 132.86 99.5) (width 0.2) (layer "F.Cu") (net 7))
 (segment (start 132.86 99.5) (end 126.5 93.14) (width 0.2) (layer "F.Cu") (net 7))
 (segment (start 127.9 92) (end 134.12 98.22) (width 0.2) (layer "F.Cu") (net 21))
 (segment (start 111.9 86.5) (end 117.4125 86.5) (width 0.2) (layer "F.Cu") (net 21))
 (segment (start 122.9125 92) (end 127.9 92) (width 0.2) (layer "F.Cu") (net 21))
 (segment (start 118.4125 87.5) (end 122.9125 92) (width 0.2) (layer "F.Cu") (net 21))
 (segment (start 117.4125 86.5) (end 118.4125 87.5) (width 0.2) (layer "F.Cu") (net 21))
 (segment (start 110.9 87.5) (end 111.9 86.5) (width 0.2) (layer "F.Cu") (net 21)))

